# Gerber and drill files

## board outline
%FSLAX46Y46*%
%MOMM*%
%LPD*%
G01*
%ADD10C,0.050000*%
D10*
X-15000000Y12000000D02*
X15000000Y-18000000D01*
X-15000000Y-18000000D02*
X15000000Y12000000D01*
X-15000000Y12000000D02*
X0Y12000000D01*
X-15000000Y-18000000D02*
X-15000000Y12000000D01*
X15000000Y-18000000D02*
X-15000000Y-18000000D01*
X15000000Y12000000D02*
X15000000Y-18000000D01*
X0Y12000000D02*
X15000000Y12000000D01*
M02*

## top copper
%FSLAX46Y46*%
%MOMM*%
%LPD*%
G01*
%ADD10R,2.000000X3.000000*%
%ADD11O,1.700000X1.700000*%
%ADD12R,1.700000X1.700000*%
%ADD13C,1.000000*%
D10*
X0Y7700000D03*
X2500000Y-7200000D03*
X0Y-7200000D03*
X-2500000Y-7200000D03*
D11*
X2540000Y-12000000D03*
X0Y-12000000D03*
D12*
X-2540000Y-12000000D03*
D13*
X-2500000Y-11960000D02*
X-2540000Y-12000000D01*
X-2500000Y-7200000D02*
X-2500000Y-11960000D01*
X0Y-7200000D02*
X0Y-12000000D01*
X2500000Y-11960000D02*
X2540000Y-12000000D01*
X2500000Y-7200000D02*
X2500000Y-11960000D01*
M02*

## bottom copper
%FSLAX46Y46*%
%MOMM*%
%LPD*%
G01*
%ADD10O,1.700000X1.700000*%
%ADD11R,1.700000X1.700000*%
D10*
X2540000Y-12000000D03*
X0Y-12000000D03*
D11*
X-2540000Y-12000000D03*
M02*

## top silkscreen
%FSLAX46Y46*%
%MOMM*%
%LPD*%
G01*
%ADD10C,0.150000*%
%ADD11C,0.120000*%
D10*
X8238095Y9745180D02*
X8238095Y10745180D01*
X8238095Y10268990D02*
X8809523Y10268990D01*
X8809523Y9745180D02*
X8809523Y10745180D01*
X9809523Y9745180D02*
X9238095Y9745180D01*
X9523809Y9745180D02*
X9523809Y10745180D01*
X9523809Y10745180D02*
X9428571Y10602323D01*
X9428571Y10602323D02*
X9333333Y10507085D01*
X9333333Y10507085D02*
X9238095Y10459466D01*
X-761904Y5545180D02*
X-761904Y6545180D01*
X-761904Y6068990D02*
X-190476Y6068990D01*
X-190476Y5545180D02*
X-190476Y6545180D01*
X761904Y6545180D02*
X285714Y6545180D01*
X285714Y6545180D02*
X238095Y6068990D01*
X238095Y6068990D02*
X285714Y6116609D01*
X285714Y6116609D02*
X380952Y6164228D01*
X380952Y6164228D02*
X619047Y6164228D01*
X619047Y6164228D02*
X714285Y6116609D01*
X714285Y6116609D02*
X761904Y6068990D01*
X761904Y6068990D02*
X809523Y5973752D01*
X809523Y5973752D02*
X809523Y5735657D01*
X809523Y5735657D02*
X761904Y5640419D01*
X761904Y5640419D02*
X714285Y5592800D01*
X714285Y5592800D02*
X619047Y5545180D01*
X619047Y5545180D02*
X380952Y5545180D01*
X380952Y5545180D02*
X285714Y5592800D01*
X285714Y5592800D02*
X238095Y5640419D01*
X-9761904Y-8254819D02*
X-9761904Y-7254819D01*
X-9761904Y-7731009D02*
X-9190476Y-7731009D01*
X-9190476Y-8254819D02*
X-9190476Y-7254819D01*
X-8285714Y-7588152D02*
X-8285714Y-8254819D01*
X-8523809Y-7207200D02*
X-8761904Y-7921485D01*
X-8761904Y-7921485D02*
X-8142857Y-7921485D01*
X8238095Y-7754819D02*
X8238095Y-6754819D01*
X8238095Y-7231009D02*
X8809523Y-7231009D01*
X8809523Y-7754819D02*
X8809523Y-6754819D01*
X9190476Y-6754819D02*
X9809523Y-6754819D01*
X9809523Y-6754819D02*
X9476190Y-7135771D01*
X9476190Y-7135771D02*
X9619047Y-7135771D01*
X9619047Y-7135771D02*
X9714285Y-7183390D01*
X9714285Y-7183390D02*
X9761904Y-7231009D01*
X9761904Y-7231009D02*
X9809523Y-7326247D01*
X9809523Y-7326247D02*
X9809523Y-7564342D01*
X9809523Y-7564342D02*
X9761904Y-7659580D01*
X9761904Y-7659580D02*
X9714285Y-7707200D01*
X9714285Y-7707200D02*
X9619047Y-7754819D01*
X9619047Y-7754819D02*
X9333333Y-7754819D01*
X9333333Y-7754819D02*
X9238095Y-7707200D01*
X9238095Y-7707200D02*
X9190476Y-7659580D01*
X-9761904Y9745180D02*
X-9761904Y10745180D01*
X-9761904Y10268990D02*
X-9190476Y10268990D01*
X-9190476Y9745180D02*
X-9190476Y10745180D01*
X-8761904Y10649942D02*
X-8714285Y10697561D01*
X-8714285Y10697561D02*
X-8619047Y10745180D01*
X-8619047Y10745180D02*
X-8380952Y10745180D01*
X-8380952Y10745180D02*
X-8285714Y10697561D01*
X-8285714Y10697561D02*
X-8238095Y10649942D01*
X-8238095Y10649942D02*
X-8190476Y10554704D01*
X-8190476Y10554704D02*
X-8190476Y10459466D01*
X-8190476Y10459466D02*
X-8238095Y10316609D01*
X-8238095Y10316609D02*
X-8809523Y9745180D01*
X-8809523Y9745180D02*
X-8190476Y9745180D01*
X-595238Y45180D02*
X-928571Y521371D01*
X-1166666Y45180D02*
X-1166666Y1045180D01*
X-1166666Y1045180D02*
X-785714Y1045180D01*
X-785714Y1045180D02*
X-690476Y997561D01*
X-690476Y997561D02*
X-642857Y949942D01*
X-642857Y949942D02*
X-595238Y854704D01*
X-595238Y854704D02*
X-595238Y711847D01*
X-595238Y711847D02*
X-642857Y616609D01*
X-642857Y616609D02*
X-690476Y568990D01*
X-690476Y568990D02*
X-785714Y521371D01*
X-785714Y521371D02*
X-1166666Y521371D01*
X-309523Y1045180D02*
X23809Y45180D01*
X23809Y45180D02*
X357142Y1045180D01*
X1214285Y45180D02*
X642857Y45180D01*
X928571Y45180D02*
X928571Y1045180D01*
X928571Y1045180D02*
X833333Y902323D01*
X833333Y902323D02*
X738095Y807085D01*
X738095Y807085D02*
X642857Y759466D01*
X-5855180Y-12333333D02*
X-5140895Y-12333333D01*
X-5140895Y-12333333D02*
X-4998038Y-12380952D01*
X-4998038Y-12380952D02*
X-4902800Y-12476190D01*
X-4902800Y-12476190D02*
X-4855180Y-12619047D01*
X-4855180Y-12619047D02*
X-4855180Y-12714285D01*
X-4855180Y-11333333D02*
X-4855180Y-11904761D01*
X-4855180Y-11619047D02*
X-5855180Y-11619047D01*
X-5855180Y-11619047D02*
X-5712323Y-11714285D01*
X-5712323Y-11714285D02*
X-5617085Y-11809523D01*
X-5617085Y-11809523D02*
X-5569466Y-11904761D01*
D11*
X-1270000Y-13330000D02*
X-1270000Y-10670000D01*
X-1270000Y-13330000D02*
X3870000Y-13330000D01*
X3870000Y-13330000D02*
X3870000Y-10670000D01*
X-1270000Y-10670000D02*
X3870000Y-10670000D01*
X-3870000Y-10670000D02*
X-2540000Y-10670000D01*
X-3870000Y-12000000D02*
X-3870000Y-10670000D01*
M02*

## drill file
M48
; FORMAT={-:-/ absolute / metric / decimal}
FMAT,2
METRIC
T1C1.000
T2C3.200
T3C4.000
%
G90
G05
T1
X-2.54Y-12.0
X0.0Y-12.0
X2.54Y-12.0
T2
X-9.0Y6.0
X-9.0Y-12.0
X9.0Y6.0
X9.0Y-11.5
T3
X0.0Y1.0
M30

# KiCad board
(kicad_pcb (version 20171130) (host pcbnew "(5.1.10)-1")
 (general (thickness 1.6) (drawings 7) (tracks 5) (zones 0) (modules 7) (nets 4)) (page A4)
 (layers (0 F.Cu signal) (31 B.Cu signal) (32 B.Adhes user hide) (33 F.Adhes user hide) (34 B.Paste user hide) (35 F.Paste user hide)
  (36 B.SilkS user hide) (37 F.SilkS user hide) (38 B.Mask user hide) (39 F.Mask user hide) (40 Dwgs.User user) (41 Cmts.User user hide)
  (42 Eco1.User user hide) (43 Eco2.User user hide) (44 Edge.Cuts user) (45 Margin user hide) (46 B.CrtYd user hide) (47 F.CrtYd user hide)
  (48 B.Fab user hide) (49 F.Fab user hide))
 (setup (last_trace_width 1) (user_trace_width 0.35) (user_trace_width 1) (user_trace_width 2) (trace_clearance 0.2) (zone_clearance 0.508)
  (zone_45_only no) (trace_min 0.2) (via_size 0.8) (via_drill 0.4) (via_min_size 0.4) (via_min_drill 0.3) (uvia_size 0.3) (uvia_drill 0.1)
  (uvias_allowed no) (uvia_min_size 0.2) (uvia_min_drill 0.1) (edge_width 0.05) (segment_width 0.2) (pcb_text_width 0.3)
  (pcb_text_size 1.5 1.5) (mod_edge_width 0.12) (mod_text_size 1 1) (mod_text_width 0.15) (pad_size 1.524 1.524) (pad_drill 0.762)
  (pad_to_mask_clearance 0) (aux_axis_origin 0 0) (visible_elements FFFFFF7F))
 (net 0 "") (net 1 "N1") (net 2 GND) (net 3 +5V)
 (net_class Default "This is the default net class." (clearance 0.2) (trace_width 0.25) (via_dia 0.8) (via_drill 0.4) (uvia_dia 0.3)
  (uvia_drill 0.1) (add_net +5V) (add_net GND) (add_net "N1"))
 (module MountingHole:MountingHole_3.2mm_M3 (layer F.Cu) (at 9 -6)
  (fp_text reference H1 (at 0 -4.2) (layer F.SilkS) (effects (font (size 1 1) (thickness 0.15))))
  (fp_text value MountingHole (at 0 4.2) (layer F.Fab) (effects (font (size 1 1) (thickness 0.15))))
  (pad 1 np_thru_hole circle (at 0 0) (size 3.2 3.2) (drill 3.2) (layers *.Cu *.Mask)))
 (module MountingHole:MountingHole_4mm (layer F.Cu) (at 0 -1)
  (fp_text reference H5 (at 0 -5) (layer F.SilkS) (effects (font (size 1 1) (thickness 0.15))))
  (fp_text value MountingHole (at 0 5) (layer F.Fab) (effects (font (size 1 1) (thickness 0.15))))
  (pad 1 np_thru_hole circle (at 0 0) (size 4 4) (drill 4) (layers *.Cu *.Mask)))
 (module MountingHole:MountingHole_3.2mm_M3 (layer F.Cu) (at -9 12)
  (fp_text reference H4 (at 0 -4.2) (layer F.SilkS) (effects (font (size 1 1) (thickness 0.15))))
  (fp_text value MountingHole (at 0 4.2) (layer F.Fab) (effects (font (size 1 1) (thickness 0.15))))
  (pad 1 np_thru_hole circle (at 0 0) (size 3.2 3.2) (drill 3.2) (layers *.Cu *.Mask)))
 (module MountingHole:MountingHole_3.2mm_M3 (layer F.Cu) (at 9 11.5)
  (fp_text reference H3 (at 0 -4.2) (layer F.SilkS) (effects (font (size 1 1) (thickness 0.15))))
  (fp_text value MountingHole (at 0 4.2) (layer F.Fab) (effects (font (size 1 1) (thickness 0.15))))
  (pad 1 np_thru_hole circle (at 0 0) (size 3.2 3.2) (drill 3.2) (layers *.Cu *.Mask)))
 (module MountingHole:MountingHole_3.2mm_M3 (layer F.Cu) (at -9 -6)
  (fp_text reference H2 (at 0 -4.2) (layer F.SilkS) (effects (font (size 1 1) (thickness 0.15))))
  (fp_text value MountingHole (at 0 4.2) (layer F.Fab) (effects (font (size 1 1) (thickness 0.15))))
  (pad 1 np_thru_hole circle (at 0 0) (size 3.2 3.2) (drill 3.2) (layers *.Cu *.Mask)))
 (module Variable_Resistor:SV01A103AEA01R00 (layer F.Cu) (at 0 -1)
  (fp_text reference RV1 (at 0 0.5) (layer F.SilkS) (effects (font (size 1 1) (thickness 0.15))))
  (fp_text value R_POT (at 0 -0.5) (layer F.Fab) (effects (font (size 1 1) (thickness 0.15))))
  (pad 2 smd rect (at 0 -6.7) (size 2 3) (layers F.Cu F.Paste F.Mask) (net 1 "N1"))
  (pad 3 smd rect (at 2.5 8.2) (size 2 3) (layers F.Cu F.Paste F.Mask) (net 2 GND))
  (pad 2 smd rect (at 0 8.2) (size 2 3) (layers F.Cu F.Paste F.Mask) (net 1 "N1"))
  (pad 1 smd rect (at -2.5 8.2) (size 2 3) (layers F.Cu F.Paste F.Mask) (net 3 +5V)))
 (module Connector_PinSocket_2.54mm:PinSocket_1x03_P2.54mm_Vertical (layer F.Cu) (at 0 12 90)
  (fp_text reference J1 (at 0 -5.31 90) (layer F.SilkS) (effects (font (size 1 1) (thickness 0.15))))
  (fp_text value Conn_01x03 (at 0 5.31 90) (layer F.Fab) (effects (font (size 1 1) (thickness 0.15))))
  (fp_line (start -1.33 -1.27) (end 1.33 -1.27) (layer F.SilkS) (width 0.12))
  (fp_line (start -1.33 -1.27) (end -1.33 3.87) (layer F.SilkS) (width 0.12))
  (fp_line (start -1.33 3.87) (end 1.33 3.87) (layer F.SilkS) (width 0.12))
  (fp_line (start 1.33 -1.27) (end 1.33 3.87) (layer F.SilkS) (width 0.12))
  (fp_line (start 1.33 -3.87) (end 1.33 -2.54) (layer F.SilkS) (width 0.12))
  (fp_line (start 0 -3.87) (end 1.33 -3.87) (layer F.SilkS) (width 0.12))
  (pad 3 thru_hole oval (at 0 2.54 90) (size 1.7 1.7) (drill 1) (layers *.Cu *.Mask) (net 2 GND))
  (pad 2 thru_hole oval (at 0 0 90) (size 1.7 1.7) (drill 1) (layers *.Cu *.Mask) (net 1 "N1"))
  (pad 1 thru_hole rect (at 0 -2.54 90) (size 1.7 1.7) (drill 1) (layers *.Cu *.Mask) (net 3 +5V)))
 (gr_line (start -15 -12) (end 15 18) (layer Edge.Cuts) (width 0.05))
 (gr_line (start -15 18) (end 15 -12) (layer Edge.Cuts) (width 0.05))
 (gr_line (start -15 -12) (end 0 -12) (layer Edge.Cuts) (width 0.05))
 (gr_line (start -15 18) (end -15 -12) (layer Edge.Cuts) (width 0.05))
 (gr_line (start 15 18) (end -15 18) (layer Edge.Cuts) (width 0.05))
 (gr_line (start 15 -12) (end 15 18) (layer Edge.Cuts) (width 0.05))
 (gr_line (start 0 -12) (end 15 -12) (layer Edge.Cuts) (width 0.05))
 (segment (start -2.5 11.96) (end -2.54 12) (width 1) (layer F.Cu) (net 3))
 (segment (start -2.5 7.2) (end -2.5 11.96) (width 1) (layer F.Cu) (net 3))
 (segment (start 0 7.2) (end 0 12) (width 1) (layer F.Cu) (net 1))
 (segment (start 2.5 11.96) (end 2.54 12) (width 1) (layer F.Cu) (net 2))
 (segment (start 2.5 7.2) (end 2.5 11.96) (width 1) (layer F.Cu) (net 2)))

